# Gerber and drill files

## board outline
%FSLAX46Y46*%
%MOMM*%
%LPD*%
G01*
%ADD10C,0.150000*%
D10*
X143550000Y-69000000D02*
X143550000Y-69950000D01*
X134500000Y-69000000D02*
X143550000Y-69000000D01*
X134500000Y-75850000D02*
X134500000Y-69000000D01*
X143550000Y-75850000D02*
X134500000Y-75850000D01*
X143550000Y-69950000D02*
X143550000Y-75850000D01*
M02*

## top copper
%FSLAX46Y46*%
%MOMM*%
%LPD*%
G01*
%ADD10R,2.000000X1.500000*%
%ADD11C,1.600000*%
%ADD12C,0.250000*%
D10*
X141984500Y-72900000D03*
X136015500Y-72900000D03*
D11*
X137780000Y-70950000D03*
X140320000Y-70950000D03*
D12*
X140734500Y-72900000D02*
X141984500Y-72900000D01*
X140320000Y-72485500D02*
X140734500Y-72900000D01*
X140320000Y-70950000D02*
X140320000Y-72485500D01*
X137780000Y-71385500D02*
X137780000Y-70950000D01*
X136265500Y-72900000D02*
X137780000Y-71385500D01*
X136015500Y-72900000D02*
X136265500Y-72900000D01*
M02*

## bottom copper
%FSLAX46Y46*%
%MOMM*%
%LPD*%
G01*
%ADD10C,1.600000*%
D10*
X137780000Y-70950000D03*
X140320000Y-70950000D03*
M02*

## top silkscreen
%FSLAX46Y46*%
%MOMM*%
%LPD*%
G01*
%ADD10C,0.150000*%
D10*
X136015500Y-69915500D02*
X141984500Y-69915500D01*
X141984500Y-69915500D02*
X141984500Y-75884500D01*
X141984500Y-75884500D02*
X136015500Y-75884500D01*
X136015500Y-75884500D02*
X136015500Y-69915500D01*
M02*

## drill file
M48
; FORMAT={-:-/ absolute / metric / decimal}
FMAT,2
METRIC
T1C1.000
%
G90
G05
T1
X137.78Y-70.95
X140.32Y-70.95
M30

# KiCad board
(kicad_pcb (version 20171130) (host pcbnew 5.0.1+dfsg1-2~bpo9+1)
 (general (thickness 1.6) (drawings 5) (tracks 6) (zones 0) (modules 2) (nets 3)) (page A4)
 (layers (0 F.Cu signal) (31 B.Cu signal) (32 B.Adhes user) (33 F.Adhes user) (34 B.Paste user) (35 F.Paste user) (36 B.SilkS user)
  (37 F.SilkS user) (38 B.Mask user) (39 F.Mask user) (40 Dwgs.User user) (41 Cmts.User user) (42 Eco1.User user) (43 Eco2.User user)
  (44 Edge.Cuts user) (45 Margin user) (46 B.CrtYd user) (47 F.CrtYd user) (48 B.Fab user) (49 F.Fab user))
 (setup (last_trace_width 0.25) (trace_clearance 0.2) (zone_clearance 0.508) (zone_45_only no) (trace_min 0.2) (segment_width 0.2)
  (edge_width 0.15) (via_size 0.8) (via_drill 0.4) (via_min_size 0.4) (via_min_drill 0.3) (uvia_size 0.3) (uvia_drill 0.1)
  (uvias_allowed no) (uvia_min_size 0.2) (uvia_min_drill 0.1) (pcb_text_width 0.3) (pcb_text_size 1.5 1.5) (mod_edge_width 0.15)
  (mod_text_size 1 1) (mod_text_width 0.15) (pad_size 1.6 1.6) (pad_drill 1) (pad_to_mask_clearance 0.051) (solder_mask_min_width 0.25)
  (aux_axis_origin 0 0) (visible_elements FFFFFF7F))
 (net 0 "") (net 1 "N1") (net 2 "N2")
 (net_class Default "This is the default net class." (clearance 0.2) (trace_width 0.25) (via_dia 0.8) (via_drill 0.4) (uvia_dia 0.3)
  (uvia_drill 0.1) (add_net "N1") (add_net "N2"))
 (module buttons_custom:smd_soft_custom (layer F.Cu) (at 139 72.9)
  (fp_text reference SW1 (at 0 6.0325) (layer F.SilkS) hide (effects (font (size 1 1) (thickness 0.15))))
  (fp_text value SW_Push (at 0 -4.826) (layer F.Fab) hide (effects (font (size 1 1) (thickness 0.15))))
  (fp_line (start -2.9845 -2.9845) (end 2.9845 -2.9845) (layer F.SilkS) (width 0.15))
  (fp_line (start 2.9845 -2.9845) (end 2.9845 2.9845) (layer F.SilkS) (width 0.15))
  (fp_line (start 2.9845 2.9845) (end -2.9845 2.9845) (layer F.SilkS) (width 0.15))
  (fp_line (start -2.9845 2.9845) (end -2.9845 -2.9845) (layer F.SilkS) (width 0.15))
  (pad 1 smd rect (at 2.9845 0 90) (size 1.5 2) (layers F.Cu F.Paste F.Mask) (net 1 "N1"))
  (pad 2 smd rect (at -2.9845 0 90) (size 1.5 2) (layers F.Cu F.Paste F.Mask) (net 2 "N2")))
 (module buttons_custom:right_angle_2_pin (layer F.Cu) (at 139.05 70.95)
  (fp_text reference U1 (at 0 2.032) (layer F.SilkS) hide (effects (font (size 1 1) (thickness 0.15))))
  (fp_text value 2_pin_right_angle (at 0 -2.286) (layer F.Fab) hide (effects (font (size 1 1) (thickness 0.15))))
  (pad 1 thru_hole circle (at -1.27 0) (size 1.6 1.6) (drill 1) (layers *.Cu *.Mask) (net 2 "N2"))
  (pad 2 thru_hole circle (at 1.27 0) (size 1.6 1.6) (drill 1) (layers *.Cu *.Mask) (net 1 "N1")))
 (gr_line (start 143.55 69) (end 143.55 69.95) (layer Edge.Cuts) (width 0.15))
 (gr_line (start 134.5 69) (end 143.55 69) (layer Edge.Cuts) (width 0.15))
 (gr_line (start 134.5 75.85) (end 134.5 69) (layer Edge.Cuts) (width 0.15))
 (gr_line (start 143.55 75.85) (end 134.5 75.85) (layer Edge.Cuts) (width 0.15))
 (gr_line (start 143.55 69.95) (end 143.55 75.85) (layer Edge.Cuts) (width 0.15))
 (segment (start 140.7345 72.9) (end 141.9845 72.9) (width 0.25) (layer F.Cu) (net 1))
 (segment (start 140.32 72.4855) (end 140.7345 72.9) (width 0.25) (layer F.Cu) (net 1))
 (segment (start 140.32 70.95) (end 140.32 72.4855) (width 0.25) (layer F.Cu) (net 1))
 (segment (start 137.78 71.3855) (end 137.78 70.95) (width 0.25) (layer F.Cu) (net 2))
 (segment (start 136.2655 72.9) (end 137.78 71.3855) (width 0.25) (layer F.Cu) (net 2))
 (segment (start 136.0155 72.9) (end 136.2655 72.9) (width 0.25) (layer F.Cu) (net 2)))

